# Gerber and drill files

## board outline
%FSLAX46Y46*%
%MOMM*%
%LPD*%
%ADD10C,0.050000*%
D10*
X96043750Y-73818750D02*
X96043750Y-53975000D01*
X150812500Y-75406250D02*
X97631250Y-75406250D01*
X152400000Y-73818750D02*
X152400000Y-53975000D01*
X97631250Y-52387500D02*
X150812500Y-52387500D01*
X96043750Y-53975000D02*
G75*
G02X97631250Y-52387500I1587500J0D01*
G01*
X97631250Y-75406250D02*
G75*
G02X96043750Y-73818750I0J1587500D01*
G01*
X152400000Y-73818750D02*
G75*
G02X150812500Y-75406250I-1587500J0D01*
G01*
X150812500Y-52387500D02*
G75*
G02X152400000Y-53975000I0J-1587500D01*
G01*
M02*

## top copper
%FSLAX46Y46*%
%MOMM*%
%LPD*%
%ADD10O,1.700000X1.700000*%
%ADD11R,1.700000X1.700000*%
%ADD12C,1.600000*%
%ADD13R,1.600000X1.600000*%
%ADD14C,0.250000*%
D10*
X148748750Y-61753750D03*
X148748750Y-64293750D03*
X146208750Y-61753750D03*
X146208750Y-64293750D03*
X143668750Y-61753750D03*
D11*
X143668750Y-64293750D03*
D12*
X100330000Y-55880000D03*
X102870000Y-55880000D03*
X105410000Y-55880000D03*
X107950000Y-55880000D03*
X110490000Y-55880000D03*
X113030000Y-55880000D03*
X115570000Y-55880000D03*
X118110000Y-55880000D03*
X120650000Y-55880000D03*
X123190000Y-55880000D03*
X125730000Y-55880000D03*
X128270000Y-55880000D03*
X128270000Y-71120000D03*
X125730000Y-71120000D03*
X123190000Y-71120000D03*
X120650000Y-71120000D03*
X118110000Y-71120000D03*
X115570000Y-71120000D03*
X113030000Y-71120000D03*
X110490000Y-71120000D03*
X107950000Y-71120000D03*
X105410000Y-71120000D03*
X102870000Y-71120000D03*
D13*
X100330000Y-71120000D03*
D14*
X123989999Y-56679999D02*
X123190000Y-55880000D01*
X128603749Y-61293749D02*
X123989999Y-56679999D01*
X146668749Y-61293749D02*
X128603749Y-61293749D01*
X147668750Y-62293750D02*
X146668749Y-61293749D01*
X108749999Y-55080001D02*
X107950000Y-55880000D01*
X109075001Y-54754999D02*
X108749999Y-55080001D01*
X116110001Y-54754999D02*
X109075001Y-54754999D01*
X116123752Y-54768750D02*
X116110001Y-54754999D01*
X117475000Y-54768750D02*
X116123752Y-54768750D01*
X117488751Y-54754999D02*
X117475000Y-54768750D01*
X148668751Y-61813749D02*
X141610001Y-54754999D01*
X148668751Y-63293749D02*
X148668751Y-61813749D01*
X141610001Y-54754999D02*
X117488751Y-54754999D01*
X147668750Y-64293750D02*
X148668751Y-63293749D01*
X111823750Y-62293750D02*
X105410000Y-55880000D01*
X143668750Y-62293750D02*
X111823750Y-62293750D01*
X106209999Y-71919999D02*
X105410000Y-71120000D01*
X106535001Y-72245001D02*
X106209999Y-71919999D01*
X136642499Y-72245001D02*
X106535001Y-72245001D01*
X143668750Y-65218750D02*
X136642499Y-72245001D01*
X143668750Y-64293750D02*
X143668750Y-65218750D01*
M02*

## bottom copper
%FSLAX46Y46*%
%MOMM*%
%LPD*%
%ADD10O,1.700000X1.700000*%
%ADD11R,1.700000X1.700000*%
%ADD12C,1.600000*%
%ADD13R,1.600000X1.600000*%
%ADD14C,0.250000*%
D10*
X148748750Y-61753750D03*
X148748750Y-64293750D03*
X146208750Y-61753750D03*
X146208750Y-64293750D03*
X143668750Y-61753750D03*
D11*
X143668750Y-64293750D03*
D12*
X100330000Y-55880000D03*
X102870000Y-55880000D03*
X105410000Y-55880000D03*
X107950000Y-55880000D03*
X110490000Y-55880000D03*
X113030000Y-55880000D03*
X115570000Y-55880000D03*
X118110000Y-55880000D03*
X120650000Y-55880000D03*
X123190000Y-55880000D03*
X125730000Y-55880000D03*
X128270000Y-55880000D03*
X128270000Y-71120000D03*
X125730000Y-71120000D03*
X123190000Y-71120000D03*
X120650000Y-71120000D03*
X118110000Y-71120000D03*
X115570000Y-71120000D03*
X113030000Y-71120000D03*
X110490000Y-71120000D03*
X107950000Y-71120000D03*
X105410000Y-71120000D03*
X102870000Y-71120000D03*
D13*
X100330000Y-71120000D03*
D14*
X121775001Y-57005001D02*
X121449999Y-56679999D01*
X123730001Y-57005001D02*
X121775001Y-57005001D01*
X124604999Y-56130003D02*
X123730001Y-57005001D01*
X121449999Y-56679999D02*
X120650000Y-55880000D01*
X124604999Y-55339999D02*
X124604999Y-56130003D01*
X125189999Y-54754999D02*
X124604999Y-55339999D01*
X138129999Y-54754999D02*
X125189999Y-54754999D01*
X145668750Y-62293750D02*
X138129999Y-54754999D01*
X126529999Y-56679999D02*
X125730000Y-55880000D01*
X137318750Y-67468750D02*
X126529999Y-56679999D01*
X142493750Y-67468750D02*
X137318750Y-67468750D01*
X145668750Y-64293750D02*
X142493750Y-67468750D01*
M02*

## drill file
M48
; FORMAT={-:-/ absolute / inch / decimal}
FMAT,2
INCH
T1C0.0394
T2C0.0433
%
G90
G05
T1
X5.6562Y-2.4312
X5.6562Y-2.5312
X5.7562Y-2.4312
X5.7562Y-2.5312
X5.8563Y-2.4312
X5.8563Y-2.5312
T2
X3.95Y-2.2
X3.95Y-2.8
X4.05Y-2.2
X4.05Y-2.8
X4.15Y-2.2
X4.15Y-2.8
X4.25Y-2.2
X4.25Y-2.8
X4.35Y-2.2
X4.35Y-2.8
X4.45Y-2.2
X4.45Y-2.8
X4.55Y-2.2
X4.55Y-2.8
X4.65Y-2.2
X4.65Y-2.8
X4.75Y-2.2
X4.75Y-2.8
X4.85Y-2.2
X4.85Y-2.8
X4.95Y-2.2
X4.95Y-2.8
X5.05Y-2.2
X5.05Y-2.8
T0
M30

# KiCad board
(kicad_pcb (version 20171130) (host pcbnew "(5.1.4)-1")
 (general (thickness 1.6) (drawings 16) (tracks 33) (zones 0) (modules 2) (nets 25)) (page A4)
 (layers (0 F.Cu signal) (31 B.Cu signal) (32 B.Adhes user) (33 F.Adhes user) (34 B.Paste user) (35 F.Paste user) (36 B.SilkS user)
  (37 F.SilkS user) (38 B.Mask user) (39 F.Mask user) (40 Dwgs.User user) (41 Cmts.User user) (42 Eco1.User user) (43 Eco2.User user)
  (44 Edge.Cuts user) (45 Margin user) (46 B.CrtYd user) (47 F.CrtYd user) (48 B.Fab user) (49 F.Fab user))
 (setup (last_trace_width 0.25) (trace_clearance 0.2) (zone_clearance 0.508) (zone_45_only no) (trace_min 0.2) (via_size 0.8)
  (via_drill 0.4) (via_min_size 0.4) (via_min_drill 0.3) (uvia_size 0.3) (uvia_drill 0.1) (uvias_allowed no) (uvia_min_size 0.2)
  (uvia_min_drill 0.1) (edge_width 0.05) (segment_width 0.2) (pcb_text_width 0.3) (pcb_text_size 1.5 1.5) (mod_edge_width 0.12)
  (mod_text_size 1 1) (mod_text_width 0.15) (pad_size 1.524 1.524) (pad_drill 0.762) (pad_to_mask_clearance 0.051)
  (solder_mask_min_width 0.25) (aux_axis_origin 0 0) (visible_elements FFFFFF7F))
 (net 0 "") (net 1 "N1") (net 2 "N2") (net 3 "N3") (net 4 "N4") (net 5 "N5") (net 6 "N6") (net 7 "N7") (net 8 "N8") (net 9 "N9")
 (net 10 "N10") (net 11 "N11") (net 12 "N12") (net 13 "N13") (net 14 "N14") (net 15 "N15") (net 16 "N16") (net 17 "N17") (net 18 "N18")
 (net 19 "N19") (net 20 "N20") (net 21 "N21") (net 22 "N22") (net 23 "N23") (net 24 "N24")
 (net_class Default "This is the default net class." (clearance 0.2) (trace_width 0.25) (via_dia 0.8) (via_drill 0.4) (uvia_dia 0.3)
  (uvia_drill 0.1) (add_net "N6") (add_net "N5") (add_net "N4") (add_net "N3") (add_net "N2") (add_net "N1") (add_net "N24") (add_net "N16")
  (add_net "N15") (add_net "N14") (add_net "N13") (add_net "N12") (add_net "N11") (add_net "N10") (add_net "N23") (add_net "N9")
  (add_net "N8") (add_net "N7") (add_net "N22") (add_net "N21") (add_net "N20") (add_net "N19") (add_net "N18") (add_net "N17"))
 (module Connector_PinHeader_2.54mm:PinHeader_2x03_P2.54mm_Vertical (layer F.Cu) (at 143.66875 64.29375 90)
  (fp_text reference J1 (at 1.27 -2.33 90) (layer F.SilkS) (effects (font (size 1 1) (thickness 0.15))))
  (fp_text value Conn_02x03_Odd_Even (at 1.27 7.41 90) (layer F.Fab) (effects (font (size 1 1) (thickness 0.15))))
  (pad 6 thru_hole oval (at 2.54 5.08 90) (size 1.7 1.7) (drill 1) (layers *.Cu *.Mask) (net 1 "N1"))
  (pad 5 thru_hole oval (at 0 5.08 90) (size 1.7 1.7) (drill 1) (layers *.Cu *.Mask) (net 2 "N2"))
  (pad 4 thru_hole oval (at 2.54 2.54 90) (size 1.7 1.7) (drill 1) (layers *.Cu *.Mask) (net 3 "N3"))
  (pad 3 thru_hole oval (at 0 2.54 90) (size 1.7 1.7) (drill 1) (layers *.Cu *.Mask) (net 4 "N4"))
  (pad 2 thru_hole oval (at 2.54 0 90) (size 1.7 1.7) (drill 1) (layers *.Cu *.Mask) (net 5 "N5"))
  (pad 1 thru_hole rect (at 0 0 90) (size 1.7 1.7) (drill 1) (layers *.Cu *.Mask) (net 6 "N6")))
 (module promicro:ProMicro (layer F.Cu) (at 114.3 63.5)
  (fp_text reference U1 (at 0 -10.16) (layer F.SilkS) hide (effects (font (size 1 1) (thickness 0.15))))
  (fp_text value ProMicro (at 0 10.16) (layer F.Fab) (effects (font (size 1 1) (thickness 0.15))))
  (pad 24 thru_hole circle (at -13.97 -7.62) (size 1.6 1.6) (drill 1.1) (layers *.Cu *.Mask F.SilkS) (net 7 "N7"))
  (pad 23 thru_hole circle (at -11.43 -7.62) (size 1.6 1.6) (drill 1.1) (layers *.Cu *.Mask F.SilkS) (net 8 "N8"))
  (pad 22 thru_hole circle (at -8.89 -7.62) (size 1.6 1.6) (drill 1.1) (layers *.Cu *.Mask F.SilkS) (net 5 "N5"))
  (pad 21 thru_hole circle (at -6.35 -7.62) (size 1.6 1.6) (drill 1.1) (layers *.Cu *.Mask F.SilkS) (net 2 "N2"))
  (pad 20 thru_hole circle (at -3.81 -7.62) (size 1.6 1.6) (drill 1.1) (layers *.Cu *.Mask F.SilkS) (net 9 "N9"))
  (pad 19 thru_hole circle (at -1.27 -7.62) (size 1.6 1.6) (drill 1.1) (layers *.Cu *.Mask F.SilkS) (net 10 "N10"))
  (pad 18 thru_hole circle (at 1.27 -7.62) (size 1.6 1.6) (drill 1.1) (layers *.Cu *.Mask F.SilkS) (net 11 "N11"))
  (pad 17 thru_hole circle (at 3.81 -7.62) (size 1.6 1.6) (drill 1.1) (layers *.Cu *.Mask F.SilkS) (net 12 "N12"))
  (pad 16 thru_hole circle (at 6.35 -7.62) (size 1.6 1.6) (drill 1.1) (layers *.Cu *.Mask F.SilkS) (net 3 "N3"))
  (pad 15 thru_hole circle (at 8.89 -7.62) (size 1.6 1.6) (drill 1.1) (layers *.Cu *.Mask F.SilkS) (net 1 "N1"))
  (pad 14 thru_hole circle (at 11.43 -7.62) (size 1.6 1.6) (drill 1.1) (layers *.Cu *.Mask F.SilkS) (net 4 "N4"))
  (pad 13 thru_hole circle (at 13.97 -7.62) (size 1.6 1.6) (drill 1.1) (layers *.Cu *.Mask F.SilkS) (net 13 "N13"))
  (pad 12 thru_hole circle (at 13.97 7.62) (size 1.6 1.6) (drill 1.1) (layers *.Cu *.Mask F.SilkS) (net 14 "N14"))
  (pad 11 thru_hole circle (at 11.43 7.62) (size 1.6 1.6) (drill 1.1) (layers *.Cu *.Mask F.SilkS) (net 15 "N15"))
  (pad 10 thru_hole circle (at 8.89 7.62) (size 1.6 1.6) (drill 1.1) (layers *.Cu *.Mask F.SilkS) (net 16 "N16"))
  (pad 9 thru_hole circle (at 6.35 7.62) (size 1.6 1.6) (drill 1.1) (layers *.Cu *.Mask F.SilkS) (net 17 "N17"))
  (pad 8 thru_hole circle (at 3.81 7.62) (size 1.6 1.6) (drill 1.1) (layers *.Cu *.Mask F.SilkS) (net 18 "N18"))
  (pad 7 thru_hole circle (at 1.27 7.62) (size 1.6 1.6) (drill 1.1) (layers *.Cu *.Mask F.SilkS) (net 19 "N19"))
  (pad 6 thru_hole circle (at -1.27 7.62) (size 1.6 1.6) (drill 1.1) (layers *.Cu *.Mask F.SilkS) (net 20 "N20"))
  (pad 5 thru_hole circle (at -3.81 7.62) (size 1.6 1.6) (drill 1.1) (layers *.Cu *.Mask F.SilkS) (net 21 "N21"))
  (pad 4 thru_hole circle (at -6.35 7.62) (size 1.6 1.6) (drill 1.1) (layers *.Cu *.Mask F.SilkS) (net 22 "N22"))
  (pad 3 thru_hole circle (at -8.89 7.62) (size 1.6 1.6) (drill 1.1) (layers *.Cu *.Mask F.SilkS) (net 6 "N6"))
  (pad 2 thru_hole circle (at -11.43 7.62) (size 1.6 1.6) (drill 1.1) (layers *.Cu *.Mask F.SilkS) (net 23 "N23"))
  (pad 1 thru_hole rect (at -13.97 7.62) (size 1.6 1.6) (drill 1.1) (layers *.Cu *.Mask F.SilkS) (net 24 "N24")))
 (gr_line (start 96.04375 73.81875) (end 96.04375 53.975) (layer Edge.Cuts) (width 0.05))
 (gr_line (start 150.8125 75.40625) (end 97.63125 75.40625) (layer Edge.Cuts) (width 0.05))
 (gr_line (start 152.4 73.81875) (end 152.4 53.975) (layer Edge.Cuts) (width 0.05))
 (gr_line (start 97.63125 52.3875) (end 150.8125 52.3875) (layer Edge.Cuts) (width 0.05))
 (gr_arc (start 97.63125 53.975) (end 97.63125 52.3875) (angle -90) (layer Edge.Cuts) (width 0.05))
 (gr_arc (start 97.63125 73.81875) (end 96.04375 73.81875) (angle -90) (layer Edge.Cuts) (width 0.05))
 (gr_arc (start 150.8125 73.81875) (end 150.8125 75.40625) (angle -90) (layer Edge.Cuts) (width 0.05))
 (gr_arc (start 150.8125 53.975) (end 152.4 53.975) (angle -90) (layer Edge.Cuts) (width 0.05))
 (segment (start 123.989999 56.679999) (end 123.19 55.88) (width 0.25) (layer F.Cu) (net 1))
 (segment (start 128.603749 61.293749) (end 123.989999 56.679999) (width 0.25) (layer F.Cu) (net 1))
 (segment (start 146.668749 61.293749) (end 128.603749 61.293749) (width 0.25) (layer F.Cu) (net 1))
 (segment (start 147.66875 62.29375) (end 146.668749 61.293749) (width 0.25) (layer F.Cu) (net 1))
 (segment (start 108.749999 55.080001) (end 107.95 55.88) (width 0.25) (layer F.Cu) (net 2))
 (segment (start 109.075001 54.754999) (end 108.749999 55.080001) (width 0.25) (layer F.Cu) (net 2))
 (segment (start 116.110001 54.754999) (end 109.075001 54.754999) (width 0.25) (layer F.Cu) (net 2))
 (segment (start 116.123752 54.76875) (end 116.110001 54.754999) (width 0.25) (layer F.Cu) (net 2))
 (segment (start 117.475 54.76875) (end 116.123752 54.76875) (width 0.25) (layer F.Cu) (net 2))
 (segment (start 117.488751 54.754999) (end 117.475 54.76875) (width 0.25) (layer F.Cu) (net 2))
 (segment (start 148.668751 61.813749) (end 141.610001 54.754999) (width 0.25) (layer F.Cu) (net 2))
 (segment (start 148.668751 63.293749) (end 148.668751 61.813749) (width 0.25) (layer F.Cu) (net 2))
 (segment (start 141.610001 54.754999) (end 117.488751 54.754999) (width 0.25) (layer F.Cu) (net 2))
 (segment (start 147.66875 64.29375) (end 148.668751 63.293749) (width 0.25) (layer F.Cu) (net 2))
 (segment (start 121.775001 57.005001) (end 121.449999 56.679999) (width 0.25) (layer B.Cu) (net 3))
 (segment (start 123.730001 57.005001) (end 121.775001 57.005001) (width 0.25) (layer B.Cu) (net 3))
 (segment (start 124.604999 56.130003) (end 123.730001 57.005001) (width 0.25) (layer B.Cu) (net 3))
 (segment (start 121.449999 56.679999) (end 120.65 55.88) (width 0.25) (layer B.Cu) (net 3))
 (segment (start 124.604999 55.339999) (end 124.604999 56.130003) (width 0.25) (layer B.Cu) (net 3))
 (segment (start 125.189999 54.754999) (end 124.604999 55.339999) (width 0.25) (layer B.Cu) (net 3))
 (segment (start 138.129999 54.754999) (end 125.189999 54.754999) (width 0.25) (layer B.Cu) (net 3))
 (segment (start 145.66875 62.29375) (end 138.129999 54.754999) (width 0.25) (layer B.Cu) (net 3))
 (segment (start 126.529999 56.679999) (end 125.73 55.88) (width 0.25) (layer B.Cu) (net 4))
 (segment (start 137.31875 67.46875) (end 126.529999 56.679999) (width 0.25) (layer B.Cu) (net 4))
 (segment (start 142.49375 67.46875) (end 137.31875 67.46875) (width 0.25) (layer B.Cu) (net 4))
 (segment (start 145.66875 64.29375) (end 142.49375 67.46875) (width 0.25) (layer B.Cu) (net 4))
 (segment (start 111.82375 62.29375) (end 105.41 55.88) (width 0.25) (layer F.Cu) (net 5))
 (segment (start 143.66875 62.29375) (end 111.82375 62.29375) (width 0.25) (layer F.Cu) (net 5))
 (segment (start 106.209999 71.919999) (end 105.41 71.12) (width 0.25) (layer F.Cu) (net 6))
 (segment (start 106.535001 72.245001) (end 106.209999 71.919999) (width 0.25) (layer F.Cu) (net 6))
 (segment (start 136.642499 72.245001) (end 106.535001 72.245001) (width 0.25) (layer F.Cu) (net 6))
 (segment (start 143.66875 65.21875) (end 136.642499 72.245001) (width 0.25) (layer F.Cu) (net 6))
 (segment (start 143.66875 64.29375) (end 143.66875 65.21875) (width 0.25) (layer F.Cu) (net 6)))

